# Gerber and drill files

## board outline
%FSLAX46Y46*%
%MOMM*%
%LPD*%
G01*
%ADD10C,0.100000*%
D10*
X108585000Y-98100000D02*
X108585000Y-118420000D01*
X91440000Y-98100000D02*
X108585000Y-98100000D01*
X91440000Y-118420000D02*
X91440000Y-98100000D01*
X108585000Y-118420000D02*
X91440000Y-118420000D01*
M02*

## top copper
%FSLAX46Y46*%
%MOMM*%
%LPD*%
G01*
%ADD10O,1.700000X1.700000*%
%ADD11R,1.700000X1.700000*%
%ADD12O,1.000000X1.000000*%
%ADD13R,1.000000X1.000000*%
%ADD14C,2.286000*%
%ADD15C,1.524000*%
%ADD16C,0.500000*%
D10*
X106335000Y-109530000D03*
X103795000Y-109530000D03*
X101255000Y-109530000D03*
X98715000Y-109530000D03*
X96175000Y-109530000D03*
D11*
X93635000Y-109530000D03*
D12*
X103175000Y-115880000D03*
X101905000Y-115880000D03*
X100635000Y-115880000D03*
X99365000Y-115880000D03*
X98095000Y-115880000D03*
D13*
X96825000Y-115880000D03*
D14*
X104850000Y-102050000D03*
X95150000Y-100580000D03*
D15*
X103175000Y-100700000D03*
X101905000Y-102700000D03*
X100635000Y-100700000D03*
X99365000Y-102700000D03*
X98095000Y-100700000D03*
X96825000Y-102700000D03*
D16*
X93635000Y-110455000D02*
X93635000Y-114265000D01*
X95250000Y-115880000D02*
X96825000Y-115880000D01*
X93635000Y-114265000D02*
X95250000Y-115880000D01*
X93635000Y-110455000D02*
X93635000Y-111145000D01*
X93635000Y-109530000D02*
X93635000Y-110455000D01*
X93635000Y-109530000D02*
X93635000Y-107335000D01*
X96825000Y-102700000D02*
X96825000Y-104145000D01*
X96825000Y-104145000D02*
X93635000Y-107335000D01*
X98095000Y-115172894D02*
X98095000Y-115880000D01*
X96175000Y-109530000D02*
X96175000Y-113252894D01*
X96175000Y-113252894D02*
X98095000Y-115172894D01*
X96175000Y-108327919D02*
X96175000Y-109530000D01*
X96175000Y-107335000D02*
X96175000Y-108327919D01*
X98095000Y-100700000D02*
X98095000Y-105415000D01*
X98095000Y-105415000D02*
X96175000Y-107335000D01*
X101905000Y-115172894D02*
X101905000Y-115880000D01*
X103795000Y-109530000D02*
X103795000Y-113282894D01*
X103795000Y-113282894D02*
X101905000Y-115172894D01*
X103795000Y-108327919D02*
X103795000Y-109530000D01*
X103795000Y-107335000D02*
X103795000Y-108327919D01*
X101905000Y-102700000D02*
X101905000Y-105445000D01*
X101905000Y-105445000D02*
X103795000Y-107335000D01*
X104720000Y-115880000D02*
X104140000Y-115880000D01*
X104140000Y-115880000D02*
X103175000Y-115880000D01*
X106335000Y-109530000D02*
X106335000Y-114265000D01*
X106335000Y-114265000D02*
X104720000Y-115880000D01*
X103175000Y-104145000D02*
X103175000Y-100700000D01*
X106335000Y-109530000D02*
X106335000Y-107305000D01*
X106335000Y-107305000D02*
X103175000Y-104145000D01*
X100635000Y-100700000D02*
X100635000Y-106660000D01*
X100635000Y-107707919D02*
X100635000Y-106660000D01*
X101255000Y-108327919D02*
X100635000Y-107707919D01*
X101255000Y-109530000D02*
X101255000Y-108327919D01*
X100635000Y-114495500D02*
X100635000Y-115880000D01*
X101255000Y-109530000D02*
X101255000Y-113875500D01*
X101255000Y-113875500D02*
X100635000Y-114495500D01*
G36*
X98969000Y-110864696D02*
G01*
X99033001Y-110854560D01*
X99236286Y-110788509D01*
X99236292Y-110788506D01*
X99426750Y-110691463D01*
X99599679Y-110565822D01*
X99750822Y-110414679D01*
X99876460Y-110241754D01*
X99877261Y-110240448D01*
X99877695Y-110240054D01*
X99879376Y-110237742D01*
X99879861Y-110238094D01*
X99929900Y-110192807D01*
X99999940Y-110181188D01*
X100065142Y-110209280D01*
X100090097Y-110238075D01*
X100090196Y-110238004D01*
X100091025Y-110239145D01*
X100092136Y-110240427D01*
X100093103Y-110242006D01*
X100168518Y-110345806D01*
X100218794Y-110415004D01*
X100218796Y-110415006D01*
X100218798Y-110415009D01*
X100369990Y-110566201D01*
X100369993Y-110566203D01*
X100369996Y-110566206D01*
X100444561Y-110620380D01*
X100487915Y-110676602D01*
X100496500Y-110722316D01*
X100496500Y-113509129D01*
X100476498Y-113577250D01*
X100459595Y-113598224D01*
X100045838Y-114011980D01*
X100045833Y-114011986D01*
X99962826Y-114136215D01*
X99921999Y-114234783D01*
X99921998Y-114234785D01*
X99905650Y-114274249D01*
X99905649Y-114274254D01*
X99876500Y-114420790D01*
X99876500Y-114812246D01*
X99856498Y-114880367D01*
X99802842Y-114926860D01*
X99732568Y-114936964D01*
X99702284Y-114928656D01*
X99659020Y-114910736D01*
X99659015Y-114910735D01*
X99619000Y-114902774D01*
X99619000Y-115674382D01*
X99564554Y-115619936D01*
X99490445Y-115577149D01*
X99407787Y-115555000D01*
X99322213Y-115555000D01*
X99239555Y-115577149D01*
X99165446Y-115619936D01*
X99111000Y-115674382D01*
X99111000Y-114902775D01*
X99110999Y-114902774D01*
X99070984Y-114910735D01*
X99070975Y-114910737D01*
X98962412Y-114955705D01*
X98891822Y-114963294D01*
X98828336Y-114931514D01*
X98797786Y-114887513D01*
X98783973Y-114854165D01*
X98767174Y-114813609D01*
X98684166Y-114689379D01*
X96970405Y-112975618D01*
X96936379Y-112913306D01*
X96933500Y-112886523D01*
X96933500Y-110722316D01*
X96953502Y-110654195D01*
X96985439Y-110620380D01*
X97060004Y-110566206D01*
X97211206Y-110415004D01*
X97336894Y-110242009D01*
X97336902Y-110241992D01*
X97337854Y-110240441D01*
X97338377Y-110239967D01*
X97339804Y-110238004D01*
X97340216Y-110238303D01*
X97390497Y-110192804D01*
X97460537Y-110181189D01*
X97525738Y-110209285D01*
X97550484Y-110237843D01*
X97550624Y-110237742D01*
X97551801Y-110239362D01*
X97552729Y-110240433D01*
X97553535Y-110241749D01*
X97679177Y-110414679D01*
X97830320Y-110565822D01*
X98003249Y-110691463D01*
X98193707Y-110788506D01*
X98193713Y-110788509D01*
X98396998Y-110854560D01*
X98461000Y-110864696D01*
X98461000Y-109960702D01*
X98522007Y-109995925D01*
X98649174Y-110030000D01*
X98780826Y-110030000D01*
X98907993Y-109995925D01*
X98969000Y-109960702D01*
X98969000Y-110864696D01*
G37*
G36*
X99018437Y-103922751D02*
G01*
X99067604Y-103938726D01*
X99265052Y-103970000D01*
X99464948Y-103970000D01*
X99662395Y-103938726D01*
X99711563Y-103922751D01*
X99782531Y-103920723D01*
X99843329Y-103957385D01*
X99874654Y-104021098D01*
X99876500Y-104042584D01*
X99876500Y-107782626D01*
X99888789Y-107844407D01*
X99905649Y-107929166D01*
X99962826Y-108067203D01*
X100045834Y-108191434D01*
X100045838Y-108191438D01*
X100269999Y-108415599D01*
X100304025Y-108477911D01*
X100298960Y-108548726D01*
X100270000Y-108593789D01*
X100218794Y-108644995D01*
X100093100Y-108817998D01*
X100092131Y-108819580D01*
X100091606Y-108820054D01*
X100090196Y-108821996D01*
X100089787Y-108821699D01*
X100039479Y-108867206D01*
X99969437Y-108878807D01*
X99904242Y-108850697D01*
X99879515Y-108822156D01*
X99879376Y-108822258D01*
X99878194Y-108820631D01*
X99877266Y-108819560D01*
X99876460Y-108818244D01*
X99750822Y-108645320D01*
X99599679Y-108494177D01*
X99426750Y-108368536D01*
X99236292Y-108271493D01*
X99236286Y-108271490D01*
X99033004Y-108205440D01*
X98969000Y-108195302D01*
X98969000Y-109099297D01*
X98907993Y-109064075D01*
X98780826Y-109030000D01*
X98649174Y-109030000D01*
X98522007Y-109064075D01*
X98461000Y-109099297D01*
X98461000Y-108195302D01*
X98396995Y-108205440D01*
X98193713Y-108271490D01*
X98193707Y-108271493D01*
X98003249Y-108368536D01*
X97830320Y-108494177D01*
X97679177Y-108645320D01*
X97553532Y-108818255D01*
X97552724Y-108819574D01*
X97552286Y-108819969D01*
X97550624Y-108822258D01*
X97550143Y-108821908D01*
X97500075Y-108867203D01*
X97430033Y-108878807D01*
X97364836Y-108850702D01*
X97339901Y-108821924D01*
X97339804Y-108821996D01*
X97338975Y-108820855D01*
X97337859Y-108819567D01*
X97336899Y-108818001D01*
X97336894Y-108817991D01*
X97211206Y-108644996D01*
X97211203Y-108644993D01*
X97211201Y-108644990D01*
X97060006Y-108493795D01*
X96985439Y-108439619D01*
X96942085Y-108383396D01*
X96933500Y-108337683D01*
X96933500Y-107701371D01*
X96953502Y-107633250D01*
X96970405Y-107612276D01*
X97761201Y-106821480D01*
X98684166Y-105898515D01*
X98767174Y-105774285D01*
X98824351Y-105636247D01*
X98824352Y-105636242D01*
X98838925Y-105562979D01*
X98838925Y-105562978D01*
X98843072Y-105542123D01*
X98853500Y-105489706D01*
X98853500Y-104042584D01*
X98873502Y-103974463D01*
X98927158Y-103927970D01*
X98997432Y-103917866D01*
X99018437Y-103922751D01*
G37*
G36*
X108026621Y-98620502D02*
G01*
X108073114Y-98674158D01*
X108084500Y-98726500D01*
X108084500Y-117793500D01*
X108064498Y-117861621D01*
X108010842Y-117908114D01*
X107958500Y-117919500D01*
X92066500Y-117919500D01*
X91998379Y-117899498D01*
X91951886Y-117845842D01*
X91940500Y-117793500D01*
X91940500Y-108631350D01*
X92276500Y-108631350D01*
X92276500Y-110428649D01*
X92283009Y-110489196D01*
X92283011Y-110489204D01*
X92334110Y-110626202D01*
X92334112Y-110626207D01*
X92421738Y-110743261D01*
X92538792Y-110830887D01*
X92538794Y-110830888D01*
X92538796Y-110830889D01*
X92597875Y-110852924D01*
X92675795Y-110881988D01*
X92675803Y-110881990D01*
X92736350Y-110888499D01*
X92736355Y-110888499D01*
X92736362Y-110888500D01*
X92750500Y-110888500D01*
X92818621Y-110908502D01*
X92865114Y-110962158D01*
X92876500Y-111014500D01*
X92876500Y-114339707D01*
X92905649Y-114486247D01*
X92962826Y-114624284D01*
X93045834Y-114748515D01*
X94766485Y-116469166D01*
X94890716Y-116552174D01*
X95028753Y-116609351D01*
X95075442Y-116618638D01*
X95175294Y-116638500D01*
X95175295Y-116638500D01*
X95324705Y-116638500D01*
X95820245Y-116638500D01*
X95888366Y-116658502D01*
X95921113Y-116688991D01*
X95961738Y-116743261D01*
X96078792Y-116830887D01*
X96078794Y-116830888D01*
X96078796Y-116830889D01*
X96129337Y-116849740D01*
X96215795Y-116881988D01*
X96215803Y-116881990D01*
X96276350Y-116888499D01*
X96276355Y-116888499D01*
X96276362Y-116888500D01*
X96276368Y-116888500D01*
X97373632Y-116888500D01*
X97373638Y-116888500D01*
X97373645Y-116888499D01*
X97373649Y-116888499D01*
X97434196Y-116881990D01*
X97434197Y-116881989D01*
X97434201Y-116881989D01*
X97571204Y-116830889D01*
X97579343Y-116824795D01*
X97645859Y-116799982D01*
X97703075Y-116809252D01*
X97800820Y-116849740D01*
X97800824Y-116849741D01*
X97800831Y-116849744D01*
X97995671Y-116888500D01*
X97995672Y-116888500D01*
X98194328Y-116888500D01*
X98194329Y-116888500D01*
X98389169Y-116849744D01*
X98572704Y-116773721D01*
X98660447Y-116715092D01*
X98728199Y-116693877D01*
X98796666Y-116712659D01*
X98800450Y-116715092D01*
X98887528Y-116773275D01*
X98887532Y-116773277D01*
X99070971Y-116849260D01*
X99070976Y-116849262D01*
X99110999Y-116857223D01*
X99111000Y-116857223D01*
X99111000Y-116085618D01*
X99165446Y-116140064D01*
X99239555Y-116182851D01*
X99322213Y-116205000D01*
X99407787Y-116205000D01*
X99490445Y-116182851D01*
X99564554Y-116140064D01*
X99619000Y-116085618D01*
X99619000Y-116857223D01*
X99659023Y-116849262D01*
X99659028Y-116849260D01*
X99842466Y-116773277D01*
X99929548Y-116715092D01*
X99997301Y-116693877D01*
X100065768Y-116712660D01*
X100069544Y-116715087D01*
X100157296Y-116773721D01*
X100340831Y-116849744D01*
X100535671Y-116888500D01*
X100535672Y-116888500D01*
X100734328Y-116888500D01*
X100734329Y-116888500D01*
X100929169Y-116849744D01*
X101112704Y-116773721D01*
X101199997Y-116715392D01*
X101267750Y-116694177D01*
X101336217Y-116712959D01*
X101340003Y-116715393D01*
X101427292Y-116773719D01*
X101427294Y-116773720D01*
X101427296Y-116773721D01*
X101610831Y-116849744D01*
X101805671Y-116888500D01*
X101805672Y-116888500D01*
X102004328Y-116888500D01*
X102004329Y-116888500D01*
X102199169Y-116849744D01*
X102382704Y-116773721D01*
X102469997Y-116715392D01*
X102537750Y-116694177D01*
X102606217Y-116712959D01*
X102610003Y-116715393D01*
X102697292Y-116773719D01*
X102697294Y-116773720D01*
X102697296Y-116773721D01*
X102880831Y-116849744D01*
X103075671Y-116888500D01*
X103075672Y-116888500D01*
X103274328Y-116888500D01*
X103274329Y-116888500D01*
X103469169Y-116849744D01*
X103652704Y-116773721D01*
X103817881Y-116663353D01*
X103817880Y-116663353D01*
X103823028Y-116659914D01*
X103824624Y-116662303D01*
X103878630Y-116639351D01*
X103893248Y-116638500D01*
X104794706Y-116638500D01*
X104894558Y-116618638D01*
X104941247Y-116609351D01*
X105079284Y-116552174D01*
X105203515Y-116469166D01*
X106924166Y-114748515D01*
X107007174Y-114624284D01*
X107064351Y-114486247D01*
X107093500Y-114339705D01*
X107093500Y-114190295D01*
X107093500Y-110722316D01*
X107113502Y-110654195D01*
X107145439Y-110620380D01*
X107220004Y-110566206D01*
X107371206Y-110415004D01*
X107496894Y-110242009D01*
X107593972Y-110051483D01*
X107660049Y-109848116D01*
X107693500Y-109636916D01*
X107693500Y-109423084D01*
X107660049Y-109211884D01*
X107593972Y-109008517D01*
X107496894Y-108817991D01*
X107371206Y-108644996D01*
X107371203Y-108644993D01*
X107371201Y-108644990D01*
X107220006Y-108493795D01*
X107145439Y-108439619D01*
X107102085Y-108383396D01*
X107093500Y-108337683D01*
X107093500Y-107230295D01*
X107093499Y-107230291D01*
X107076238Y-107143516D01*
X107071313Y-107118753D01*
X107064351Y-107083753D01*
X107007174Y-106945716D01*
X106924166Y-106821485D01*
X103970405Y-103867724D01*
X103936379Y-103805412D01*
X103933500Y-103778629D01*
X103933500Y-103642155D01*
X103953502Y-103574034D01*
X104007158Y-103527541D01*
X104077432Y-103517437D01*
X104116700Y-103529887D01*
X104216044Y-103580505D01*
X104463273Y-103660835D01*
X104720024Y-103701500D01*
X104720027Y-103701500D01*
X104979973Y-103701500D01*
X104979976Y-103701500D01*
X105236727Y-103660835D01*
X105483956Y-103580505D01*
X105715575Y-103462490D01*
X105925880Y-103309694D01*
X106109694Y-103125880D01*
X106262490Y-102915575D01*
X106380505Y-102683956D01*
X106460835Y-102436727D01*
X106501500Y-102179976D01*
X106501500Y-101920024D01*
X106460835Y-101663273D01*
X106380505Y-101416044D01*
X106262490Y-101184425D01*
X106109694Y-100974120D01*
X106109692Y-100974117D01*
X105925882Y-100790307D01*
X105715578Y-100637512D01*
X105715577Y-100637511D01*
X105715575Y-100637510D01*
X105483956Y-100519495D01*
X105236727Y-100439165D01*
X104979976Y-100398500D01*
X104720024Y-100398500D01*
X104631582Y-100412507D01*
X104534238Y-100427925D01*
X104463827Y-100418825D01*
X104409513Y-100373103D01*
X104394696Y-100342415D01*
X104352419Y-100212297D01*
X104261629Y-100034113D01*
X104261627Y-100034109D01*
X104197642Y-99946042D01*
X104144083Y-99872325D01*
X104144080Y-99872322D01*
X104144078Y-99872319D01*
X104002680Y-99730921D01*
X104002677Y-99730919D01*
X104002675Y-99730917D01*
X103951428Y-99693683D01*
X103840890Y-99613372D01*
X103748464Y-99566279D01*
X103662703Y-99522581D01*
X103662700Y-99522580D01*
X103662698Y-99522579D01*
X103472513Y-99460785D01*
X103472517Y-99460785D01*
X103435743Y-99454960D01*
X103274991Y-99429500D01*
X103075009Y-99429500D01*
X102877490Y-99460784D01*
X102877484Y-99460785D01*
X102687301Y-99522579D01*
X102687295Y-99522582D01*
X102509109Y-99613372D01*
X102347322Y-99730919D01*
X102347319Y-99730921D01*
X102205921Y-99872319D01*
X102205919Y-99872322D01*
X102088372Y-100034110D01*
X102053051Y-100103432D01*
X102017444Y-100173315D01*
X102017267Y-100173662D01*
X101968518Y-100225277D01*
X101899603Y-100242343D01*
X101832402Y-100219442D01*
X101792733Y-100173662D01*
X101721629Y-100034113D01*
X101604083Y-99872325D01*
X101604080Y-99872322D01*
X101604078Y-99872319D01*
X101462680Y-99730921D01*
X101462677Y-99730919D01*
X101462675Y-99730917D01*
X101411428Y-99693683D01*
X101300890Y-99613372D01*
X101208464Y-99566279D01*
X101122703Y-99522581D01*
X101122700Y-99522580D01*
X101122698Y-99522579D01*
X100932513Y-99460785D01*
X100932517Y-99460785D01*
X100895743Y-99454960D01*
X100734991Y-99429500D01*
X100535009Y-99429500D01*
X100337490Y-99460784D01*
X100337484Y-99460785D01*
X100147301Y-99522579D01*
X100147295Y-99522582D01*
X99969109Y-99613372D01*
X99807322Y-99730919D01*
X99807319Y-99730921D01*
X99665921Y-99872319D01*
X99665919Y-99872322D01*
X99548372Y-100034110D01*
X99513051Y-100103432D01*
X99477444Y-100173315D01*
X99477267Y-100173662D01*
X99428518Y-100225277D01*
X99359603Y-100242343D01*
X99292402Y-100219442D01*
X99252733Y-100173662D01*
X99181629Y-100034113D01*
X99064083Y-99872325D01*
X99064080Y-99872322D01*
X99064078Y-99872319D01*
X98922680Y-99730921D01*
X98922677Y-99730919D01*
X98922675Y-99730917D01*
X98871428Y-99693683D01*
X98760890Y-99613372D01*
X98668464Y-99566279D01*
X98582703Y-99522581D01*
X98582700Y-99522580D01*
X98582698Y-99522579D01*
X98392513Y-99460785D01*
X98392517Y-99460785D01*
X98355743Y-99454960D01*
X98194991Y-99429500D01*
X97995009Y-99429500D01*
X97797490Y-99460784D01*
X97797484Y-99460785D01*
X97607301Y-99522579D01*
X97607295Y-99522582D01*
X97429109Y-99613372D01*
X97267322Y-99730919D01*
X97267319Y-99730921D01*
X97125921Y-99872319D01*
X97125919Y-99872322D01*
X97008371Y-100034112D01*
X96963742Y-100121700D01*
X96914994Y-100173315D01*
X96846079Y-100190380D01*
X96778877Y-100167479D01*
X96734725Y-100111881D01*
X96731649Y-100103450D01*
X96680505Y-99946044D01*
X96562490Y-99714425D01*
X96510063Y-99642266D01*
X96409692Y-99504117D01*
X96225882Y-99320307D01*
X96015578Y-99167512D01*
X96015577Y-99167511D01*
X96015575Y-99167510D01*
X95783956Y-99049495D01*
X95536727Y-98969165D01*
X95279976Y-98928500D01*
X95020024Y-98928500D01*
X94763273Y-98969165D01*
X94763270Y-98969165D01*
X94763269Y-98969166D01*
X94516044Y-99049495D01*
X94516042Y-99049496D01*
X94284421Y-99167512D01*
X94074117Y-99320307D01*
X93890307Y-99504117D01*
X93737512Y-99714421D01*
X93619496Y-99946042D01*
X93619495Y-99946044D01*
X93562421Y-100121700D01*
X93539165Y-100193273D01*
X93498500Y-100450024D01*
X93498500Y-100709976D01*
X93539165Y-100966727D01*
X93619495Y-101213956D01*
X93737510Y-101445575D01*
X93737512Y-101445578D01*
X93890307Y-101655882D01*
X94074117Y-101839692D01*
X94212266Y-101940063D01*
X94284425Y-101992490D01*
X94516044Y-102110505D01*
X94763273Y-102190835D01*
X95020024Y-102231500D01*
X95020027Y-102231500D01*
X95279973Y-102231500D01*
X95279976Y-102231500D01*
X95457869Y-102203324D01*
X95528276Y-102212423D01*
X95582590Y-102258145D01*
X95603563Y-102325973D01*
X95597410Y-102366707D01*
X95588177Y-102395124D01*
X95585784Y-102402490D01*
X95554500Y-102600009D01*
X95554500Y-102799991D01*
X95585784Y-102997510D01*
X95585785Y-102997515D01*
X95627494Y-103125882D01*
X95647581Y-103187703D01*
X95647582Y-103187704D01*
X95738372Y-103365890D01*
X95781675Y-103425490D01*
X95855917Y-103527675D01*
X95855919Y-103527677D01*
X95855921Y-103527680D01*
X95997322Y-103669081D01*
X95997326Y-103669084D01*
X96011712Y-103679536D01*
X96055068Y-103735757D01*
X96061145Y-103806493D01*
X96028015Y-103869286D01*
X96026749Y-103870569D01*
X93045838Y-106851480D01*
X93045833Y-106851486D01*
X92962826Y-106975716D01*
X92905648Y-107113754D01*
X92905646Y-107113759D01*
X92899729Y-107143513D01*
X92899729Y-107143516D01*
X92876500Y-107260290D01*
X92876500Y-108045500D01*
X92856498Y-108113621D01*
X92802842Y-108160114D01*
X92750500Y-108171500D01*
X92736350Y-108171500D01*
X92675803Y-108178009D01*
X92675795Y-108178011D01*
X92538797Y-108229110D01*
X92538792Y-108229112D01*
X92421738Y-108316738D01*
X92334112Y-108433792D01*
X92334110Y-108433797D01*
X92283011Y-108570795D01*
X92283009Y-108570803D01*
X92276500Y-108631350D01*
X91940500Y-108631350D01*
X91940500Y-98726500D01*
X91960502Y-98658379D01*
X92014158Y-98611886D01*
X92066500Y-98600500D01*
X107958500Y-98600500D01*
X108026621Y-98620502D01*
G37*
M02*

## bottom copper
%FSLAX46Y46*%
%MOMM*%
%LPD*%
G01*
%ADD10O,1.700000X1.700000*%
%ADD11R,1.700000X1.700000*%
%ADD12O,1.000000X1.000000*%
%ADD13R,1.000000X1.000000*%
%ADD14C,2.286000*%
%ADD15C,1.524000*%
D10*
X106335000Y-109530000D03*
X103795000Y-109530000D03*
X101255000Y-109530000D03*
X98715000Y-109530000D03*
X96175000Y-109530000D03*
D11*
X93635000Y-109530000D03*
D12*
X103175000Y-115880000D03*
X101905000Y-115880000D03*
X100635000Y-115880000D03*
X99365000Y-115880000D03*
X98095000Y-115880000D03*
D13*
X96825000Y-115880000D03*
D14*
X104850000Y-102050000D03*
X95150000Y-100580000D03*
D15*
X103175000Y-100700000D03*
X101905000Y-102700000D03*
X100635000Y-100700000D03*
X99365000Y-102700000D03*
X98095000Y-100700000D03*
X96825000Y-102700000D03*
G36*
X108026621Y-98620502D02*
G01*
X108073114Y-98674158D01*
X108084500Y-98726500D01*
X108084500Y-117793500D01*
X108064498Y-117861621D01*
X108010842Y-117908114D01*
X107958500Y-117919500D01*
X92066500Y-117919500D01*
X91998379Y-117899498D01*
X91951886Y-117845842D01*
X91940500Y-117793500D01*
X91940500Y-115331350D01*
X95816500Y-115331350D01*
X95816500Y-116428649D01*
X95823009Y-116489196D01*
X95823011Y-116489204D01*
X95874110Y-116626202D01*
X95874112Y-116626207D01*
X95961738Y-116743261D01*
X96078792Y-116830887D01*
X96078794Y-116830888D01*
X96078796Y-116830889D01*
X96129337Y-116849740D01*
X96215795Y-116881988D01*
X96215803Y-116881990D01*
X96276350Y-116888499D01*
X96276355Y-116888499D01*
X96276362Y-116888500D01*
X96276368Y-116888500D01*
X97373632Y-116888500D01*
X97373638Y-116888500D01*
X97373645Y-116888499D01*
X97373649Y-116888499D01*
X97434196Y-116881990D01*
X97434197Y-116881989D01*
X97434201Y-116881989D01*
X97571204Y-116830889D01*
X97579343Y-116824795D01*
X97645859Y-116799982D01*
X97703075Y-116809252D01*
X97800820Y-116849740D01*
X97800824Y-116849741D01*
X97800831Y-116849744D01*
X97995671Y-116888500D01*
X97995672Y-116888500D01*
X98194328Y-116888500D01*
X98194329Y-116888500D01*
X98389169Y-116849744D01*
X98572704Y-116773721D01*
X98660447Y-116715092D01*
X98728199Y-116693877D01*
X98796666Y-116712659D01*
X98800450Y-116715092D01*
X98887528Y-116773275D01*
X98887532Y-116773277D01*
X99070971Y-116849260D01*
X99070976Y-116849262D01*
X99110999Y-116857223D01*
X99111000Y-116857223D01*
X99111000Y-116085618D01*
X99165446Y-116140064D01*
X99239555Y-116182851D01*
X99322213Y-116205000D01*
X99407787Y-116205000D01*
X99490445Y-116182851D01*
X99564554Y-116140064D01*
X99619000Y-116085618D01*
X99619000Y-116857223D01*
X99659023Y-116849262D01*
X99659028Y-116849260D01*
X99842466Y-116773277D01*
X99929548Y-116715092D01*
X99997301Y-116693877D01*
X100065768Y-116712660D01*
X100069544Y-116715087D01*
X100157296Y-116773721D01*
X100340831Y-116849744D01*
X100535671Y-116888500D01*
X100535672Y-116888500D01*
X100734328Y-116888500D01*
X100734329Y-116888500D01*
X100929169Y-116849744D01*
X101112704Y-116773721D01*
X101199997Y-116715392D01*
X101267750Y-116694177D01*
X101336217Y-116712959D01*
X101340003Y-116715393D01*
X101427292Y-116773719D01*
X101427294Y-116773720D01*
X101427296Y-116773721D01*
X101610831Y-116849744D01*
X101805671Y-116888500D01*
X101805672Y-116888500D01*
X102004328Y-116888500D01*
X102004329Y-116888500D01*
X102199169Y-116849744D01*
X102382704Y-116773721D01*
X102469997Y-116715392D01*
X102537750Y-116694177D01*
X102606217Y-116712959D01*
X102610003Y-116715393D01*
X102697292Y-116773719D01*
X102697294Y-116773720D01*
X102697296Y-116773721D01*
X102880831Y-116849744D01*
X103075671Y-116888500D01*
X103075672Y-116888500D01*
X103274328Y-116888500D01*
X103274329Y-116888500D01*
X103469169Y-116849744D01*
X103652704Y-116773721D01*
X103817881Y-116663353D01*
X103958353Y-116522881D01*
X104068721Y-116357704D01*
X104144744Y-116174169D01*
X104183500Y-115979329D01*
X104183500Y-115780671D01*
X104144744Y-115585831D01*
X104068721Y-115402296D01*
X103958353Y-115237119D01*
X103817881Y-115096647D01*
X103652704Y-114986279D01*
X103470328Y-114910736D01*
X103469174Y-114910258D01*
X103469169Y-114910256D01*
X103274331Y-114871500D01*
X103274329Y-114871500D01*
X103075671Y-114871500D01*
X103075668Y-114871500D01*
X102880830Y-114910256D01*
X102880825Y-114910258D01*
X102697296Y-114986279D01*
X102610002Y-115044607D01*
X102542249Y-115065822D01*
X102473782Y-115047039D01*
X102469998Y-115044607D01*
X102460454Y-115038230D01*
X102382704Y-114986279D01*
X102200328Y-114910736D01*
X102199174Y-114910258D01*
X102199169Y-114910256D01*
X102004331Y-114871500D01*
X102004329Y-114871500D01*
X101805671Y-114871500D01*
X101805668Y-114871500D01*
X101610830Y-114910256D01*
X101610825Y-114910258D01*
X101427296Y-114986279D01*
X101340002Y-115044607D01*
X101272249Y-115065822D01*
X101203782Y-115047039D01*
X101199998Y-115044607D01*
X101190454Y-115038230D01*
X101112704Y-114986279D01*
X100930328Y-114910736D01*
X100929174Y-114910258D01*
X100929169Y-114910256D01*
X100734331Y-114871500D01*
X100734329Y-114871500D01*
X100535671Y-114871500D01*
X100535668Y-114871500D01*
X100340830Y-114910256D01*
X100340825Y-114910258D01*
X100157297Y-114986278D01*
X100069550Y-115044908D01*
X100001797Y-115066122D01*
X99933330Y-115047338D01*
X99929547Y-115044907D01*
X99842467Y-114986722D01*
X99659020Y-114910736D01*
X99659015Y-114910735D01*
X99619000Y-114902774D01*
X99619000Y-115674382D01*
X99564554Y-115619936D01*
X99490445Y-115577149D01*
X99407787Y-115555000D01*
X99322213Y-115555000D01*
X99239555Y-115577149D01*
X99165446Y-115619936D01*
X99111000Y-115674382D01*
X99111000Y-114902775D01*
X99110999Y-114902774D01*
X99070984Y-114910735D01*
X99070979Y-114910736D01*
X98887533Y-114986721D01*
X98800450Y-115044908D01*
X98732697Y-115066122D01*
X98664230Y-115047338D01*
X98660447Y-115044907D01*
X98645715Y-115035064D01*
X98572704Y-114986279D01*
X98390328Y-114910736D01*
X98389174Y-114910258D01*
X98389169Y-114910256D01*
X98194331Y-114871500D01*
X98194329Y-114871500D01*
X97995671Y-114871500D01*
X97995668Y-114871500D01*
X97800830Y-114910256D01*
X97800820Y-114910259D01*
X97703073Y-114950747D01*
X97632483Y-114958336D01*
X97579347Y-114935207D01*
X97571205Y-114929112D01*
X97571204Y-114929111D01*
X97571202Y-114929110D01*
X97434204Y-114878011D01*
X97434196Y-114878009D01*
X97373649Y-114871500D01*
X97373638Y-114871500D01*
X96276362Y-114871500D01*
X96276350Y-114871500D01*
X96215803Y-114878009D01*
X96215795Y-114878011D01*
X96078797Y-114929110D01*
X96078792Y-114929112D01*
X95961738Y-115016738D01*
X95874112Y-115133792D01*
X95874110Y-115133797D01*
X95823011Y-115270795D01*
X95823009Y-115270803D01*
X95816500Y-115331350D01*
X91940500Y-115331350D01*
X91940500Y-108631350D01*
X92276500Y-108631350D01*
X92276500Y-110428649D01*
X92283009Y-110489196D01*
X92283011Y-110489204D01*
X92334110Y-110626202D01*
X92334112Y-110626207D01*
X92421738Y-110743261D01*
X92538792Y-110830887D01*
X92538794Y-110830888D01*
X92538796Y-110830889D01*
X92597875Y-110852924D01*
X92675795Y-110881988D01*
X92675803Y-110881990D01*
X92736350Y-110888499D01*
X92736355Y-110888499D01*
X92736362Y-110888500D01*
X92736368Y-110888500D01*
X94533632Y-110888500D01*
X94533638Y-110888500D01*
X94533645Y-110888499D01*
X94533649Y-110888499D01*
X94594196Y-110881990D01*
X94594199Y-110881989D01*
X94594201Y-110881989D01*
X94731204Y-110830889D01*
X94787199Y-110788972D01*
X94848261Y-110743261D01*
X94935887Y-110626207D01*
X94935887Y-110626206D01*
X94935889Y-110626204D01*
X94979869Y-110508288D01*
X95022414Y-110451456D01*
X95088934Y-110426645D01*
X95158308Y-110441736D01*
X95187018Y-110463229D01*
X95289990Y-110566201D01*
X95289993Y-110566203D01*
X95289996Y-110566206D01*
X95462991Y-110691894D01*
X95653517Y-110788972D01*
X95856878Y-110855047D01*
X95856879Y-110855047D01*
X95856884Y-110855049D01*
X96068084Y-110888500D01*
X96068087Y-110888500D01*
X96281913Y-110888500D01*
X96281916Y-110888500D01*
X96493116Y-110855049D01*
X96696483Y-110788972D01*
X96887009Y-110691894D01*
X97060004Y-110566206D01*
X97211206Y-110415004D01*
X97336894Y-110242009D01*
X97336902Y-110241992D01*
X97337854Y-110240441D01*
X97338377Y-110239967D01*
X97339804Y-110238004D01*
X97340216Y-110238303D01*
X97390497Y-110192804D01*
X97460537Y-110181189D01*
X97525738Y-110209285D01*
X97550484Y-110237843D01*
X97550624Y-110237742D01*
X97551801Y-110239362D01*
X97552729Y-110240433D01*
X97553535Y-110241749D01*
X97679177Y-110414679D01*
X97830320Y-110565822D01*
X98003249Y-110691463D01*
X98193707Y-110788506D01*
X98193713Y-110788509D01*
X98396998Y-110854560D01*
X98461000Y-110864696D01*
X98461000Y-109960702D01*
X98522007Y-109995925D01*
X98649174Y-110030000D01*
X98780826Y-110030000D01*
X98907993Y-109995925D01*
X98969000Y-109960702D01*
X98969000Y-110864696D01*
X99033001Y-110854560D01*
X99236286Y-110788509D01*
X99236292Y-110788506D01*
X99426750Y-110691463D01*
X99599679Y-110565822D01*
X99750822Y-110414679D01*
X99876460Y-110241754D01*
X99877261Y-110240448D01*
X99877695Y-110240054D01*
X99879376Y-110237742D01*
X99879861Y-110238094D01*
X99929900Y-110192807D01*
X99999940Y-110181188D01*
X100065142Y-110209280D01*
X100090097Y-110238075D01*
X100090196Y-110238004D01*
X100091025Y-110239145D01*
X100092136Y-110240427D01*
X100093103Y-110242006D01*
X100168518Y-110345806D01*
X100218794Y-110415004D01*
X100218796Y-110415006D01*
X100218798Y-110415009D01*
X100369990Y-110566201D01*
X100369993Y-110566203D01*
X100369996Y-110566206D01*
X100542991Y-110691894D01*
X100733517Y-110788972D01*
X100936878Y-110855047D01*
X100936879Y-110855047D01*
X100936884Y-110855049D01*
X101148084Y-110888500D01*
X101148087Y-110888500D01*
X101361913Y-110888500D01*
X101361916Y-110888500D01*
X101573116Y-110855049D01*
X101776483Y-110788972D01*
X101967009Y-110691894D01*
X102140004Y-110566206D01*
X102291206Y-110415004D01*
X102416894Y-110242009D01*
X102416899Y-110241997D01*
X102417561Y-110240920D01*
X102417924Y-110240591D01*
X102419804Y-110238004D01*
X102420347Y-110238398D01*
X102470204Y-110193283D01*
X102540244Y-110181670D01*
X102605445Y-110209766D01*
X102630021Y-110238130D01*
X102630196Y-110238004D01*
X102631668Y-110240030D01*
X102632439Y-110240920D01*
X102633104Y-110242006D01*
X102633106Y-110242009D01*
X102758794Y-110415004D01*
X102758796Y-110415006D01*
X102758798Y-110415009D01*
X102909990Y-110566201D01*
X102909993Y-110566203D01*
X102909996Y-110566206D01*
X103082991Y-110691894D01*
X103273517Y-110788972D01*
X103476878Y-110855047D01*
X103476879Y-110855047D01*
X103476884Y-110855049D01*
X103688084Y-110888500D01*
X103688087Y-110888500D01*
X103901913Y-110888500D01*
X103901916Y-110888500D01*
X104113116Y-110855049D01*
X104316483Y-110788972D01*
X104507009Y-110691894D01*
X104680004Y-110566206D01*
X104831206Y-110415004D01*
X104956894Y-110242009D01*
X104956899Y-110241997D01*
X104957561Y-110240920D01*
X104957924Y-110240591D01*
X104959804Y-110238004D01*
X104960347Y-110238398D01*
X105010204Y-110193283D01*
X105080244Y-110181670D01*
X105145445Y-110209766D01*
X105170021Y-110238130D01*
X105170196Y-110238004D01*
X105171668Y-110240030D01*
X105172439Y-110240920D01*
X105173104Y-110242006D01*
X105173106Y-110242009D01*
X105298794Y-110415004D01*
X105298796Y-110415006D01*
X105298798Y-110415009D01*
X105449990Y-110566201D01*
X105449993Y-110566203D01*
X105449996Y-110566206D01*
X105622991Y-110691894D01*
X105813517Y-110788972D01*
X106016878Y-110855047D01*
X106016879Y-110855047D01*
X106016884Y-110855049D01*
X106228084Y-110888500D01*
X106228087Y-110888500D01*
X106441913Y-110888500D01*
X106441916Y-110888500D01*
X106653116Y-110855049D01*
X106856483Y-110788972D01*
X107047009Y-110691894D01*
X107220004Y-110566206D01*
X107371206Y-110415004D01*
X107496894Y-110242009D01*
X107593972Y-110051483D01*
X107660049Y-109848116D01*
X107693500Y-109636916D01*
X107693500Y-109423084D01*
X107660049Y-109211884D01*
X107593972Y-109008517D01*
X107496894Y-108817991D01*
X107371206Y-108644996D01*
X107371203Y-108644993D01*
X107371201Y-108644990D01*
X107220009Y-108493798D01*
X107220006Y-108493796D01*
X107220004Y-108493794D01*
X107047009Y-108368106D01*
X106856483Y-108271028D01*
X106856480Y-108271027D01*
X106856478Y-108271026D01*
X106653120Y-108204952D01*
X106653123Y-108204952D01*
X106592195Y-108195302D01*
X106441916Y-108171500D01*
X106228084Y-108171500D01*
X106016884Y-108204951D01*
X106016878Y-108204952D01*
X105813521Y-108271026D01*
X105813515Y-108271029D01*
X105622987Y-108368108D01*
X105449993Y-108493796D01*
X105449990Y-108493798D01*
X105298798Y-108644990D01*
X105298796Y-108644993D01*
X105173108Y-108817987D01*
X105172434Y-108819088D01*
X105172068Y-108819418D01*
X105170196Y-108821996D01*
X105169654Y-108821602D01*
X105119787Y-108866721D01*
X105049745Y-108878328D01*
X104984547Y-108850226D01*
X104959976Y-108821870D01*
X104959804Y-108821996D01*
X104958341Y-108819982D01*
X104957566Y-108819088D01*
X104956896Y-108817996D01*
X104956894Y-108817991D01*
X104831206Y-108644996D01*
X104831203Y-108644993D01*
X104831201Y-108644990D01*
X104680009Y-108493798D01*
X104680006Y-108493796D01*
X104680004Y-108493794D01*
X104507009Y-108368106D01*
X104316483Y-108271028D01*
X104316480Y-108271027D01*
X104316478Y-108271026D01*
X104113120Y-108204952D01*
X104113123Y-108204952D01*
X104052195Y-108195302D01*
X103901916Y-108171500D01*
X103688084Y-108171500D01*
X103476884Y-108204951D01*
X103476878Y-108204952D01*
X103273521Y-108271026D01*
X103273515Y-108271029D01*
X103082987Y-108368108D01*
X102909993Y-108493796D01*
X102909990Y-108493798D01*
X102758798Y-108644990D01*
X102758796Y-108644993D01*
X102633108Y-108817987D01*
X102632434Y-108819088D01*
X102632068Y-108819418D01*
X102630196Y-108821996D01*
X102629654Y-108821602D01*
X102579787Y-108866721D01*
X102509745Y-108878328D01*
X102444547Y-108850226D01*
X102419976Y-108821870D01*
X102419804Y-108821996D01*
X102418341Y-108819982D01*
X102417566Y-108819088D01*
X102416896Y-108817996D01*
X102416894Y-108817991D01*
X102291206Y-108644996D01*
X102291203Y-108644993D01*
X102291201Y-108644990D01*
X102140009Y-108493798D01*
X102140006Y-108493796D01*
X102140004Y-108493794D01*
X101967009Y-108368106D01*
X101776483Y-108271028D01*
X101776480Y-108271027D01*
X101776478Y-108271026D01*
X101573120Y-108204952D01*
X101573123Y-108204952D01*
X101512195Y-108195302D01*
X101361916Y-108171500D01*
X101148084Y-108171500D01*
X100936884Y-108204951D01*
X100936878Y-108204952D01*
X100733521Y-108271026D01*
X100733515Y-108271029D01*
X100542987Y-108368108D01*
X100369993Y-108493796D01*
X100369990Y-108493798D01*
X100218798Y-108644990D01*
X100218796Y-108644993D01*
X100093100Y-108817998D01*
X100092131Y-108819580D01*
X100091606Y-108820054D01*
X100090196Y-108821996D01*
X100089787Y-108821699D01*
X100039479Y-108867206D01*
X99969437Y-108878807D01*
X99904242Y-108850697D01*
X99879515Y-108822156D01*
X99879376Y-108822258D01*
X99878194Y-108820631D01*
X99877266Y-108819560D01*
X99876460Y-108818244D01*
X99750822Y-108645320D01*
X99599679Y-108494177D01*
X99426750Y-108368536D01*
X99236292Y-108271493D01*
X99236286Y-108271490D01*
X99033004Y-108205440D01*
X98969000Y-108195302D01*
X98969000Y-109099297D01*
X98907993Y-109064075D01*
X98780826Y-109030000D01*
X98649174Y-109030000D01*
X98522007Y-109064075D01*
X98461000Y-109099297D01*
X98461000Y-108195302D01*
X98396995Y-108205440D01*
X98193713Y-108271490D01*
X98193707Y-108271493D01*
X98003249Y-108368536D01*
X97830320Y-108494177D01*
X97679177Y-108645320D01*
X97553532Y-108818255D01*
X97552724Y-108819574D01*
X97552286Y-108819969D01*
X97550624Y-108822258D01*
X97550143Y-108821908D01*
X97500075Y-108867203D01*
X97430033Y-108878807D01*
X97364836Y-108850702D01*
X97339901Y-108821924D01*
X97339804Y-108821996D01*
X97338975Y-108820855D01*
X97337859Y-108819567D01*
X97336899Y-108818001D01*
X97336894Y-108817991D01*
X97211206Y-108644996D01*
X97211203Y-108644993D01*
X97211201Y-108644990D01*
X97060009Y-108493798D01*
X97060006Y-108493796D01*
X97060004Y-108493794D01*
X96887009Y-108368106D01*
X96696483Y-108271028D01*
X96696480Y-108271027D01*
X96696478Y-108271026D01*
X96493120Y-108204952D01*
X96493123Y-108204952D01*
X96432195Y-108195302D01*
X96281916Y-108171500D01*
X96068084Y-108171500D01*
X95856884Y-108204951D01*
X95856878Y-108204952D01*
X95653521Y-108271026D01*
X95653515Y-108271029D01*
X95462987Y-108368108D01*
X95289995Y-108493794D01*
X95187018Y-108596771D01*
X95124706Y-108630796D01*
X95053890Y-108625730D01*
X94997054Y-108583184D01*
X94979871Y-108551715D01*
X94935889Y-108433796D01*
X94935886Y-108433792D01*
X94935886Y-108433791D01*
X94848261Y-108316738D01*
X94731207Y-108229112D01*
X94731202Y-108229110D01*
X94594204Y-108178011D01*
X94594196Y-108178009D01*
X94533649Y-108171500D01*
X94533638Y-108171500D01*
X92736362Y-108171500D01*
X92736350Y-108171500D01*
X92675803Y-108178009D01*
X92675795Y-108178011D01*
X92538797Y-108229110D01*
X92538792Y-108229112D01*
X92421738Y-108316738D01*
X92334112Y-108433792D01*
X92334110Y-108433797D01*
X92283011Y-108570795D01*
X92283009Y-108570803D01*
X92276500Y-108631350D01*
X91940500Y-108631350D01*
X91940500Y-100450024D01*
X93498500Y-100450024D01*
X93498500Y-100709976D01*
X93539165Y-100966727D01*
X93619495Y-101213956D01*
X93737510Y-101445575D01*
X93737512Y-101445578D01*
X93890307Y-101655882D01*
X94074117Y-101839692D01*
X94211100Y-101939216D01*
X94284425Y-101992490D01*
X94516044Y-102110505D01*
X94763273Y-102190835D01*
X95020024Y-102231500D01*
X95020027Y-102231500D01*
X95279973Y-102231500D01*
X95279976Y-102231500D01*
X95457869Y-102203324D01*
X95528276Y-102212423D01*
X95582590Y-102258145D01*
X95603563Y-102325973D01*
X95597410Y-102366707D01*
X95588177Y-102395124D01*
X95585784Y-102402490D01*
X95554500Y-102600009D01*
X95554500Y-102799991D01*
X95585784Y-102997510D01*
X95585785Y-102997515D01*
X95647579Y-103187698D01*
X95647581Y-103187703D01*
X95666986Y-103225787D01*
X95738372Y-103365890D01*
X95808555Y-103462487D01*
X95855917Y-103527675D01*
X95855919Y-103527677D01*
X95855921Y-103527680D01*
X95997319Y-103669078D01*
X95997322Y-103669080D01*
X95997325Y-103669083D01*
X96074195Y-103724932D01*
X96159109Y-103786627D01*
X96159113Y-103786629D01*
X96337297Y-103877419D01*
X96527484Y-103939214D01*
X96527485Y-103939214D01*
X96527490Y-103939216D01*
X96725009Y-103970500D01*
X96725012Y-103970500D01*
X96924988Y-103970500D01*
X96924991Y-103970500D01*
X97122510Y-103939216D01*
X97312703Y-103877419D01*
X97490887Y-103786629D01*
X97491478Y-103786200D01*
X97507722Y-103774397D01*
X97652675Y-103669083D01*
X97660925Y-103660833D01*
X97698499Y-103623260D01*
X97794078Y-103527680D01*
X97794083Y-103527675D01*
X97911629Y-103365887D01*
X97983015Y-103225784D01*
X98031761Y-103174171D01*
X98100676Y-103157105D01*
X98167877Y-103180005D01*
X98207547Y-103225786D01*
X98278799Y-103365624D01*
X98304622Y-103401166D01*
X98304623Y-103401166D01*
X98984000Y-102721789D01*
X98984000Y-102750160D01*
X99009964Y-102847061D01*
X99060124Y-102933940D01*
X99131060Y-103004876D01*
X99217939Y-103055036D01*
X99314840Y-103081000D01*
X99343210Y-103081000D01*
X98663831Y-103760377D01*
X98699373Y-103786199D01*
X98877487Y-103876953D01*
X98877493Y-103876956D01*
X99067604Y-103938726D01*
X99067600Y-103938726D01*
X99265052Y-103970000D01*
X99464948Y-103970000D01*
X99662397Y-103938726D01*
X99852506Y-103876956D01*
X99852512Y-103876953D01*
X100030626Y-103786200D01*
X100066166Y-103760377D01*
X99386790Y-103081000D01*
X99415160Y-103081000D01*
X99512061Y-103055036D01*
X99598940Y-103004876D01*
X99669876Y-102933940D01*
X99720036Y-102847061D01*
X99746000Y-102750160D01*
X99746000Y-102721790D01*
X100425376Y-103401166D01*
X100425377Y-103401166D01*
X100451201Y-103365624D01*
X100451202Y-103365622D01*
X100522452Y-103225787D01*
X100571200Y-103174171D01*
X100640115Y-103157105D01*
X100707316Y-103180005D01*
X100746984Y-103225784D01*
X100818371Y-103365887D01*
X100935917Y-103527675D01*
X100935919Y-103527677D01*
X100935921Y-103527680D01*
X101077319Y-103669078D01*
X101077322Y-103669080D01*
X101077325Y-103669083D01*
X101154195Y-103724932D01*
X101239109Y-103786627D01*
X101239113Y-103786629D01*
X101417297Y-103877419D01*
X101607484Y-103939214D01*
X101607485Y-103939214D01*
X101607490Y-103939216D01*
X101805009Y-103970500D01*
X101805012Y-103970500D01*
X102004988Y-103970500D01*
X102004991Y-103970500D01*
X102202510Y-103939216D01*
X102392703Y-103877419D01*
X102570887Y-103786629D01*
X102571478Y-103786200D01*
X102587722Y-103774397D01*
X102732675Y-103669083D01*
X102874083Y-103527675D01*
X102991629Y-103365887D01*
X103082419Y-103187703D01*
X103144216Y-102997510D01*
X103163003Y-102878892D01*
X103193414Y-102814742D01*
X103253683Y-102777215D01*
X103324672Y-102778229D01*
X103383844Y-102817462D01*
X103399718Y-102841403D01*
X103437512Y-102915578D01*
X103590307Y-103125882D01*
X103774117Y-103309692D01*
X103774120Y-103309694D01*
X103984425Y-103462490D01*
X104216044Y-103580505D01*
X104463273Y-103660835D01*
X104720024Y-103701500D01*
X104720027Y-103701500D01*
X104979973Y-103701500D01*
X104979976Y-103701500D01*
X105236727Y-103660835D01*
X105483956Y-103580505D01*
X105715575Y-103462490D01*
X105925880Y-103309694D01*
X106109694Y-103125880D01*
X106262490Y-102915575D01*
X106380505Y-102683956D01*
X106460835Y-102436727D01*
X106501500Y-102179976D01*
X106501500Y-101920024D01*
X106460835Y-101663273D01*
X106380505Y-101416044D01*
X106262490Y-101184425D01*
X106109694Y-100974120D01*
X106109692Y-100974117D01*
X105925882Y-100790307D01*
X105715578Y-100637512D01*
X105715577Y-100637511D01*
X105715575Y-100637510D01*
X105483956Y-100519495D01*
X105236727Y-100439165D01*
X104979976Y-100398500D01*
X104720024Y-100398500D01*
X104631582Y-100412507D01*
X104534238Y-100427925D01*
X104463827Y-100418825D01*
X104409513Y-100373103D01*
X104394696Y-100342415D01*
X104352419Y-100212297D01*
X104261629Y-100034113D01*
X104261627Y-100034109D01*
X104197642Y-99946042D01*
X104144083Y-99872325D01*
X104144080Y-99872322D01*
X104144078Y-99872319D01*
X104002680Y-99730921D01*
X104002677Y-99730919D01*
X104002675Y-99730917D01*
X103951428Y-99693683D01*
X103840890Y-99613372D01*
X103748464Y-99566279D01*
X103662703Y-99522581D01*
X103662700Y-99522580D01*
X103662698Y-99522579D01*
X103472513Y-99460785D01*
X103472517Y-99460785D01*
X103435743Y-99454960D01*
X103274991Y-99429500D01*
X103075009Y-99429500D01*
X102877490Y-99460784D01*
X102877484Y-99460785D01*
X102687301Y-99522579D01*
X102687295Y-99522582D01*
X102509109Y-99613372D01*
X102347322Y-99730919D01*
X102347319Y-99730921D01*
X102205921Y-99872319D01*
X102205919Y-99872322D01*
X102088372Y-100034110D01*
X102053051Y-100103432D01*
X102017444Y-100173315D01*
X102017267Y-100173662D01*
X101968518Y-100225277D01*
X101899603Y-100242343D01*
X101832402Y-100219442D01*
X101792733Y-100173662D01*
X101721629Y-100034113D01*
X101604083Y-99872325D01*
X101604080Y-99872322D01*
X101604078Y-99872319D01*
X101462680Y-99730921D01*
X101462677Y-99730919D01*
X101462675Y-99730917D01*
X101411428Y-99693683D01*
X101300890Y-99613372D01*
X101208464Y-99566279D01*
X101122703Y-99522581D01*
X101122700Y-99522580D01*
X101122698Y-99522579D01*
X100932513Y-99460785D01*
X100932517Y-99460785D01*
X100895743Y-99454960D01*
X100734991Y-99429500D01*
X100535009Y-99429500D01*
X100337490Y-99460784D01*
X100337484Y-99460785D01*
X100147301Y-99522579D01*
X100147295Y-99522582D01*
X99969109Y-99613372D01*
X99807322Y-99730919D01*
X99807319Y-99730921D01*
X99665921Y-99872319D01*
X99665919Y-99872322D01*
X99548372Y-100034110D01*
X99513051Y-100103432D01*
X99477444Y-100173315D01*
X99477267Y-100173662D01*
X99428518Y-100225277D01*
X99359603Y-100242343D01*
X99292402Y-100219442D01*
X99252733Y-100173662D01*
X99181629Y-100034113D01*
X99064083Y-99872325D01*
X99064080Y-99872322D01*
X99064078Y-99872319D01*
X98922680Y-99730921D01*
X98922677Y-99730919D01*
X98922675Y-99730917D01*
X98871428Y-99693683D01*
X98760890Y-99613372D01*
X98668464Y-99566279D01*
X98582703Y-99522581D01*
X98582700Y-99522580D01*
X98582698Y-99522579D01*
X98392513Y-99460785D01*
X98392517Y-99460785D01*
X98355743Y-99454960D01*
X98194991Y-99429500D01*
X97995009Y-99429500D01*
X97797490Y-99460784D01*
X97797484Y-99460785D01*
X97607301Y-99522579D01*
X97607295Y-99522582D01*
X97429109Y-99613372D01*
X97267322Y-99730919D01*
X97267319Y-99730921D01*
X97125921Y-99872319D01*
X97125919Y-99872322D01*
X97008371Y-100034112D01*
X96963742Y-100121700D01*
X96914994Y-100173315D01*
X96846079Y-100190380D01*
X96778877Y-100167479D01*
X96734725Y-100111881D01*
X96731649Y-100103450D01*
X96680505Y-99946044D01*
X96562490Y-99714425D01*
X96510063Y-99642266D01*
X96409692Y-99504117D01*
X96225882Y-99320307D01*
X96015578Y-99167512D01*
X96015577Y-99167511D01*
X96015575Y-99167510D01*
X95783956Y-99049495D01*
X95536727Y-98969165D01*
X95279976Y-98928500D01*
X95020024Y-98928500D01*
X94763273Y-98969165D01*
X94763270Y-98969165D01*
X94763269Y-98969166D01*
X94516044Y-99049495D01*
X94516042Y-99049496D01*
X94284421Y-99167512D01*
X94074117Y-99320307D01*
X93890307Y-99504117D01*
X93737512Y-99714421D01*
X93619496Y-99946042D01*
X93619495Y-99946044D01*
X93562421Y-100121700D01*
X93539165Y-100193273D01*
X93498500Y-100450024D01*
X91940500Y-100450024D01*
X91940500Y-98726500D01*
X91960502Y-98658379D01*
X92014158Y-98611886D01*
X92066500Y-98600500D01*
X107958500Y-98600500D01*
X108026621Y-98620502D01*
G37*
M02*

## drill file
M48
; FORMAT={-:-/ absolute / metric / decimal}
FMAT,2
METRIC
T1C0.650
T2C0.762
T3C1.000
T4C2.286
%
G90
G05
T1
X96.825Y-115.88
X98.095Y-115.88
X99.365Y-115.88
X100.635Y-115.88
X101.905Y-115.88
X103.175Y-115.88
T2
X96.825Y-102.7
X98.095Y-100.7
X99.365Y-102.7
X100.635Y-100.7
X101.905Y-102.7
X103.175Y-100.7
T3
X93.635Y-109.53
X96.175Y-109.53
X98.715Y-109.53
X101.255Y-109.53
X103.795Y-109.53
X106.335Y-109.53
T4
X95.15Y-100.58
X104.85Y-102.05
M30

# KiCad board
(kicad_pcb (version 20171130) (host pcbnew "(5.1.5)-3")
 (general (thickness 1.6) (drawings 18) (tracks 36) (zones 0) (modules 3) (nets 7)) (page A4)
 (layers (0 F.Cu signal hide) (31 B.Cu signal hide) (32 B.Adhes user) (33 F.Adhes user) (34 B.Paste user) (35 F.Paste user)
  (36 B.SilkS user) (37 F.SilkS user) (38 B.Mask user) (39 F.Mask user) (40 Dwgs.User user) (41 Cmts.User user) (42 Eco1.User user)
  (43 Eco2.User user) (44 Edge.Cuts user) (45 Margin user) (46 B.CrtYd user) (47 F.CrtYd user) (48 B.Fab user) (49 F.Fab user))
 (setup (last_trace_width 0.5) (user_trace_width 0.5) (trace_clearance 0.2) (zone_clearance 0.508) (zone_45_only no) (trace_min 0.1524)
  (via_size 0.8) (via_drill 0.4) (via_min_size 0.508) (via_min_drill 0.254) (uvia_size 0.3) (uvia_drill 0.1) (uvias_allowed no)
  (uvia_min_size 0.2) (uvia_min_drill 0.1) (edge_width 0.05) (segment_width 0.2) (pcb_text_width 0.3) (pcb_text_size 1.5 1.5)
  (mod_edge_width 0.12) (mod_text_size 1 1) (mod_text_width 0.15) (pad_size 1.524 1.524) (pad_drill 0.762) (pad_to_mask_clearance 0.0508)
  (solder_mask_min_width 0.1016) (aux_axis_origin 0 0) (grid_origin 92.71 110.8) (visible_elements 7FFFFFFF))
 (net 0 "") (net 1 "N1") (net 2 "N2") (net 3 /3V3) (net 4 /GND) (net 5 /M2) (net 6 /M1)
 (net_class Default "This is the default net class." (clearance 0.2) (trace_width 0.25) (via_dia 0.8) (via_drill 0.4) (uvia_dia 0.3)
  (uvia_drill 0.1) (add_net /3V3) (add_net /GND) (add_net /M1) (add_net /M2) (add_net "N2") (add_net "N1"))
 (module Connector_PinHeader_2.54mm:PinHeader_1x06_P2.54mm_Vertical (layer F.Cu) (at 93.635 109.53 90)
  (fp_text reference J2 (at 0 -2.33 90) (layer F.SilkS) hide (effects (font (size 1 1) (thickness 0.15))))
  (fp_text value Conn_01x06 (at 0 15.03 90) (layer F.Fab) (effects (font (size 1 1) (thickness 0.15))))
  (pad 6 thru_hole oval (at 0 12.7 90) (size 1.7 1.7) (drill 1) (layers *.Cu *.Mask) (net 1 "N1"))
  (pad 5 thru_hole oval (at 0 10.16 90) (size 1.7 1.7) (drill 1) (layers *.Cu *.Mask) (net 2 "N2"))
  (pad 4 thru_hole oval (at 0 7.62 90) (size 1.7 1.7) (drill 1) (layers *.Cu *.Mask) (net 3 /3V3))
  (pad 3 thru_hole oval (at 0 5.08 90) (size 1.7 1.7) (drill 1) (layers *.Cu *.Mask) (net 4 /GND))
  (pad 2 thru_hole oval (at 0 2.54 90) (size 1.7 1.7) (drill 1) (layers *.Cu *.Mask) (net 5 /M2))
  (pad 1 thru_hole rect (at 0 0 90) (size 1.7 1.7) (drill 1) (layers *.Cu *.Mask) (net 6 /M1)))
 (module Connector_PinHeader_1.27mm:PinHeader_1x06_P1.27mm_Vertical (layer F.Cu) (at 96.825 115.88 90)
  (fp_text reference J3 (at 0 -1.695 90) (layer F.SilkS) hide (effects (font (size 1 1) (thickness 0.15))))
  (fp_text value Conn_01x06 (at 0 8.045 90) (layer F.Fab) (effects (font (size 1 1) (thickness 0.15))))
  (pad 6 thru_hole oval (at 0 6.35 90) (size 1 1) (drill 0.65) (layers *.Cu *.Mask) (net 1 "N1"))
  (pad 5 thru_hole oval (at 0 5.08 90) (size 1 1) (drill 0.65) (layers *.Cu *.Mask) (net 2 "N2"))
  (pad 4 thru_hole oval (at 0 3.81 90) (size 1 1) (drill 0.65) (layers *.Cu *.Mask) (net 3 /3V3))
  (pad 3 thru_hole oval (at 0 2.54 90) (size 1 1) (drill 0.65) (layers *.Cu *.Mask) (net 4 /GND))
  (pad 2 thru_hole oval (at 0 1.27 90) (size 1 1) (drill 0.65) (layers *.Cu *.Mask) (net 5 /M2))
  (pad 1 thru_hole rect (at 0 0 90) (size 1 1) (drill 0.65) (layers *.Cu *.Mask) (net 6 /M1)))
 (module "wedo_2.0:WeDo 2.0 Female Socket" (layer F.Cu) (at 100 100)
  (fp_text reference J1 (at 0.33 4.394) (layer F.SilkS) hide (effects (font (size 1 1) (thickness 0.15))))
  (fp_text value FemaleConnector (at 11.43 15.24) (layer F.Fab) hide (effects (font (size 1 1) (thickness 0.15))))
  (pad "" thru_hole circle (at 4.85 2.05) (size 2.286 2.286) (drill 2.286) (layers *.Cu *.Mask))
  (pad "" thru_hole circle (at -4.85 0.58) (size 2.286 2.286) (drill 2.286) (layers *.Cu *.Mask))
  (pad 6 thru_hole circle (at 3.175 0.7) (size 1.524 1.524) (drill 0.762) (layers *.Cu *.Mask) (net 1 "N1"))
  (pad 5 thru_hole circle (at 1.905 2.7) (size 1.524 1.524) (drill 0.762) (layers *.Cu *.Mask) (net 2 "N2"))
  (pad 4 thru_hole circle (at 0.635 0.7) (size 1.524 1.524) (drill 0.762) (layers *.Cu *.Mask) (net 3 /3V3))
  (pad 3 thru_hole circle (at -0.635 2.7) (size 1.524 1.524) (drill 0.762) (layers *.Cu *.Mask) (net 4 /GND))
  (pad 2 thru_hole circle (at -1.905 0.7) (size 1.524 1.524) (drill 0.762) (layers *.Cu *.Mask) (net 5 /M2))
  (pad 1 thru_hole circle (at -3.175 2.7) (size 1.524 1.524) (drill 0.762) (layers *.Cu *.Mask) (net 6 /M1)))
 (gr_line (start 108.585 98.1) (end 108.585 118.42) (layer Edge.Cuts) (width 0.1))
 (gr_line (start 91.44 98.1) (end 108.585 98.1) (layer Edge.Cuts) (width 0.1))
 (gr_line (start 91.44 118.42) (end 91.44 98.1) (layer Edge.Cuts) (width 0.1))
 (gr_line (start 108.585 118.42) (end 91.44 118.42) (layer Edge.Cuts) (width 0.1))
 (segment (start 93.635 110.455) (end 93.635 114.265) (width 0.5) (layer F.Cu) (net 6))
 (segment (start 95.25 115.88) (end 96.825 115.88) (width 0.5) (layer F.Cu) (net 6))
 (segment (start 93.635 114.265) (end 95.25 115.88) (width 0.5) (layer F.Cu) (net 6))
 (segment (start 93.635 110.455) (end 93.635 111.145) (width 0.5) (layer F.Cu) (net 6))
 (segment (start 93.635 109.53) (end 93.635 110.455) (width 0.5) (layer F.Cu) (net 6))
 (segment (start 93.635 109.53) (end 93.635 107.335) (width 0.5) (layer F.Cu) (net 6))
 (segment (start 96.825 102.7) (end 96.825 104.145) (width 0.5) (layer F.Cu) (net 6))
 (segment (start 96.825 104.145) (end 93.635 107.335) (width 0.5) (layer F.Cu) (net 6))
 (segment (start 98.095 115.172894) (end 98.095 115.88) (width 0.5) (layer F.Cu) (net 5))
 (segment (start 96.175 109.53) (end 96.175 113.252894) (width 0.5) (layer F.Cu) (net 5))
 (segment (start 96.175 113.252894) (end 98.095 115.172894) (width 0.5) (layer F.Cu) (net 5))
 (segment (start 96.175 108.327919) (end 96.175 109.53) (width 0.5) (layer F.Cu) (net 5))
 (segment (start 96.175 107.335) (end 96.175 108.327919) (width 0.5) (layer F.Cu) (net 5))
 (segment (start 98.095 100.7) (end 98.095 105.415) (width 0.5) (layer F.Cu) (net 5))
 (segment (start 98.095 105.415) (end 96.175 107.335) (width 0.5) (layer F.Cu) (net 5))
 (segment (start 101.905 115.172894) (end 101.905 115.88) (width 0.5) (layer F.Cu) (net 2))
 (segment (start 103.795 109.53) (end 103.795 113.282894) (width 0.5) (layer F.Cu) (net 2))
 (segment (start 103.795 113.282894) (end 101.905 115.172894) (width 0.5) (layer F.Cu) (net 2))
 (segment (start 103.795 108.327919) (end 103.795 109.53) (width 0.5) (layer F.Cu) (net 2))
 (segment (start 103.795 107.335) (end 103.795 108.327919) (width 0.5) (layer F.Cu) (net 2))
 (segment (start 101.905 102.7) (end 101.905 105.445) (width 0.5) (layer F.Cu) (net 2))
 (segment (start 101.905 105.445) (end 103.795 107.335) (width 0.5) (layer F.Cu) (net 2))
 (segment (start 104.72 115.88) (end 104.14 115.88) (width 0.5) (layer F.Cu) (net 1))
 (segment (start 104.14 115.88) (end 103.175 115.88) (width 0.5) (layer F.Cu) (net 1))
 (segment (start 106.335 109.53) (end 106.335 114.265) (width 0.5) (layer F.Cu) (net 1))
 (segment (start 106.335 114.265) (end 104.72 115.88) (width 0.5) (layer F.Cu) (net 1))
 (segment (start 103.175 104.145) (end 103.175 100.7) (width 0.5) (layer F.Cu) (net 1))
 (segment (start 106.335 109.53) (end 106.335 107.305) (width 0.5) (layer F.Cu) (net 1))
 (segment (start 106.335 107.305) (end 103.175 104.145) (width 0.5) (layer F.Cu) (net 1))
 (segment (start 100.635 100.7) (end 100.635 106.66) (width 0.5) (layer F.Cu) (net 3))
 (segment (start 100.635 107.707919) (end 100.635 106.66) (width 0.5) (layer F.Cu) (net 3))
 (segment (start 101.255 108.327919) (end 100.635 107.707919) (width 0.5) (layer F.Cu) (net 3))
 (segment (start 101.255 109.53) (end 101.255 108.327919) (width 0.5) (layer F.Cu) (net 3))
 (segment (start 100.635 114.4955) (end 100.635 115.88) (width 0.5) (layer F.Cu) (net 3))
 (segment (start 101.255 109.53) (end 101.255 113.8755) (width 0.5) (layer F.Cu) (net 3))
 (segment (start 101.255 113.8755) (end 100.635 114.4955) (width 0.5) (layer F.Cu) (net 3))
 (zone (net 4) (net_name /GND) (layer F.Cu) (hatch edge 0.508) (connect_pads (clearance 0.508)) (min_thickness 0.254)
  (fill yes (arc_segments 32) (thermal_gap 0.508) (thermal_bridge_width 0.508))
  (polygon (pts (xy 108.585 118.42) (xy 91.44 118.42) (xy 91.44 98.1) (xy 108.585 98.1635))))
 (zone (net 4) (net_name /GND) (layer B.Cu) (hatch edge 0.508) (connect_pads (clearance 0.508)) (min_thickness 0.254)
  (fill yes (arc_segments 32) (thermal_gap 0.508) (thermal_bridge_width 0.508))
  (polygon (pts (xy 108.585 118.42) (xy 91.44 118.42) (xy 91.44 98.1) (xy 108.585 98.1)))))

